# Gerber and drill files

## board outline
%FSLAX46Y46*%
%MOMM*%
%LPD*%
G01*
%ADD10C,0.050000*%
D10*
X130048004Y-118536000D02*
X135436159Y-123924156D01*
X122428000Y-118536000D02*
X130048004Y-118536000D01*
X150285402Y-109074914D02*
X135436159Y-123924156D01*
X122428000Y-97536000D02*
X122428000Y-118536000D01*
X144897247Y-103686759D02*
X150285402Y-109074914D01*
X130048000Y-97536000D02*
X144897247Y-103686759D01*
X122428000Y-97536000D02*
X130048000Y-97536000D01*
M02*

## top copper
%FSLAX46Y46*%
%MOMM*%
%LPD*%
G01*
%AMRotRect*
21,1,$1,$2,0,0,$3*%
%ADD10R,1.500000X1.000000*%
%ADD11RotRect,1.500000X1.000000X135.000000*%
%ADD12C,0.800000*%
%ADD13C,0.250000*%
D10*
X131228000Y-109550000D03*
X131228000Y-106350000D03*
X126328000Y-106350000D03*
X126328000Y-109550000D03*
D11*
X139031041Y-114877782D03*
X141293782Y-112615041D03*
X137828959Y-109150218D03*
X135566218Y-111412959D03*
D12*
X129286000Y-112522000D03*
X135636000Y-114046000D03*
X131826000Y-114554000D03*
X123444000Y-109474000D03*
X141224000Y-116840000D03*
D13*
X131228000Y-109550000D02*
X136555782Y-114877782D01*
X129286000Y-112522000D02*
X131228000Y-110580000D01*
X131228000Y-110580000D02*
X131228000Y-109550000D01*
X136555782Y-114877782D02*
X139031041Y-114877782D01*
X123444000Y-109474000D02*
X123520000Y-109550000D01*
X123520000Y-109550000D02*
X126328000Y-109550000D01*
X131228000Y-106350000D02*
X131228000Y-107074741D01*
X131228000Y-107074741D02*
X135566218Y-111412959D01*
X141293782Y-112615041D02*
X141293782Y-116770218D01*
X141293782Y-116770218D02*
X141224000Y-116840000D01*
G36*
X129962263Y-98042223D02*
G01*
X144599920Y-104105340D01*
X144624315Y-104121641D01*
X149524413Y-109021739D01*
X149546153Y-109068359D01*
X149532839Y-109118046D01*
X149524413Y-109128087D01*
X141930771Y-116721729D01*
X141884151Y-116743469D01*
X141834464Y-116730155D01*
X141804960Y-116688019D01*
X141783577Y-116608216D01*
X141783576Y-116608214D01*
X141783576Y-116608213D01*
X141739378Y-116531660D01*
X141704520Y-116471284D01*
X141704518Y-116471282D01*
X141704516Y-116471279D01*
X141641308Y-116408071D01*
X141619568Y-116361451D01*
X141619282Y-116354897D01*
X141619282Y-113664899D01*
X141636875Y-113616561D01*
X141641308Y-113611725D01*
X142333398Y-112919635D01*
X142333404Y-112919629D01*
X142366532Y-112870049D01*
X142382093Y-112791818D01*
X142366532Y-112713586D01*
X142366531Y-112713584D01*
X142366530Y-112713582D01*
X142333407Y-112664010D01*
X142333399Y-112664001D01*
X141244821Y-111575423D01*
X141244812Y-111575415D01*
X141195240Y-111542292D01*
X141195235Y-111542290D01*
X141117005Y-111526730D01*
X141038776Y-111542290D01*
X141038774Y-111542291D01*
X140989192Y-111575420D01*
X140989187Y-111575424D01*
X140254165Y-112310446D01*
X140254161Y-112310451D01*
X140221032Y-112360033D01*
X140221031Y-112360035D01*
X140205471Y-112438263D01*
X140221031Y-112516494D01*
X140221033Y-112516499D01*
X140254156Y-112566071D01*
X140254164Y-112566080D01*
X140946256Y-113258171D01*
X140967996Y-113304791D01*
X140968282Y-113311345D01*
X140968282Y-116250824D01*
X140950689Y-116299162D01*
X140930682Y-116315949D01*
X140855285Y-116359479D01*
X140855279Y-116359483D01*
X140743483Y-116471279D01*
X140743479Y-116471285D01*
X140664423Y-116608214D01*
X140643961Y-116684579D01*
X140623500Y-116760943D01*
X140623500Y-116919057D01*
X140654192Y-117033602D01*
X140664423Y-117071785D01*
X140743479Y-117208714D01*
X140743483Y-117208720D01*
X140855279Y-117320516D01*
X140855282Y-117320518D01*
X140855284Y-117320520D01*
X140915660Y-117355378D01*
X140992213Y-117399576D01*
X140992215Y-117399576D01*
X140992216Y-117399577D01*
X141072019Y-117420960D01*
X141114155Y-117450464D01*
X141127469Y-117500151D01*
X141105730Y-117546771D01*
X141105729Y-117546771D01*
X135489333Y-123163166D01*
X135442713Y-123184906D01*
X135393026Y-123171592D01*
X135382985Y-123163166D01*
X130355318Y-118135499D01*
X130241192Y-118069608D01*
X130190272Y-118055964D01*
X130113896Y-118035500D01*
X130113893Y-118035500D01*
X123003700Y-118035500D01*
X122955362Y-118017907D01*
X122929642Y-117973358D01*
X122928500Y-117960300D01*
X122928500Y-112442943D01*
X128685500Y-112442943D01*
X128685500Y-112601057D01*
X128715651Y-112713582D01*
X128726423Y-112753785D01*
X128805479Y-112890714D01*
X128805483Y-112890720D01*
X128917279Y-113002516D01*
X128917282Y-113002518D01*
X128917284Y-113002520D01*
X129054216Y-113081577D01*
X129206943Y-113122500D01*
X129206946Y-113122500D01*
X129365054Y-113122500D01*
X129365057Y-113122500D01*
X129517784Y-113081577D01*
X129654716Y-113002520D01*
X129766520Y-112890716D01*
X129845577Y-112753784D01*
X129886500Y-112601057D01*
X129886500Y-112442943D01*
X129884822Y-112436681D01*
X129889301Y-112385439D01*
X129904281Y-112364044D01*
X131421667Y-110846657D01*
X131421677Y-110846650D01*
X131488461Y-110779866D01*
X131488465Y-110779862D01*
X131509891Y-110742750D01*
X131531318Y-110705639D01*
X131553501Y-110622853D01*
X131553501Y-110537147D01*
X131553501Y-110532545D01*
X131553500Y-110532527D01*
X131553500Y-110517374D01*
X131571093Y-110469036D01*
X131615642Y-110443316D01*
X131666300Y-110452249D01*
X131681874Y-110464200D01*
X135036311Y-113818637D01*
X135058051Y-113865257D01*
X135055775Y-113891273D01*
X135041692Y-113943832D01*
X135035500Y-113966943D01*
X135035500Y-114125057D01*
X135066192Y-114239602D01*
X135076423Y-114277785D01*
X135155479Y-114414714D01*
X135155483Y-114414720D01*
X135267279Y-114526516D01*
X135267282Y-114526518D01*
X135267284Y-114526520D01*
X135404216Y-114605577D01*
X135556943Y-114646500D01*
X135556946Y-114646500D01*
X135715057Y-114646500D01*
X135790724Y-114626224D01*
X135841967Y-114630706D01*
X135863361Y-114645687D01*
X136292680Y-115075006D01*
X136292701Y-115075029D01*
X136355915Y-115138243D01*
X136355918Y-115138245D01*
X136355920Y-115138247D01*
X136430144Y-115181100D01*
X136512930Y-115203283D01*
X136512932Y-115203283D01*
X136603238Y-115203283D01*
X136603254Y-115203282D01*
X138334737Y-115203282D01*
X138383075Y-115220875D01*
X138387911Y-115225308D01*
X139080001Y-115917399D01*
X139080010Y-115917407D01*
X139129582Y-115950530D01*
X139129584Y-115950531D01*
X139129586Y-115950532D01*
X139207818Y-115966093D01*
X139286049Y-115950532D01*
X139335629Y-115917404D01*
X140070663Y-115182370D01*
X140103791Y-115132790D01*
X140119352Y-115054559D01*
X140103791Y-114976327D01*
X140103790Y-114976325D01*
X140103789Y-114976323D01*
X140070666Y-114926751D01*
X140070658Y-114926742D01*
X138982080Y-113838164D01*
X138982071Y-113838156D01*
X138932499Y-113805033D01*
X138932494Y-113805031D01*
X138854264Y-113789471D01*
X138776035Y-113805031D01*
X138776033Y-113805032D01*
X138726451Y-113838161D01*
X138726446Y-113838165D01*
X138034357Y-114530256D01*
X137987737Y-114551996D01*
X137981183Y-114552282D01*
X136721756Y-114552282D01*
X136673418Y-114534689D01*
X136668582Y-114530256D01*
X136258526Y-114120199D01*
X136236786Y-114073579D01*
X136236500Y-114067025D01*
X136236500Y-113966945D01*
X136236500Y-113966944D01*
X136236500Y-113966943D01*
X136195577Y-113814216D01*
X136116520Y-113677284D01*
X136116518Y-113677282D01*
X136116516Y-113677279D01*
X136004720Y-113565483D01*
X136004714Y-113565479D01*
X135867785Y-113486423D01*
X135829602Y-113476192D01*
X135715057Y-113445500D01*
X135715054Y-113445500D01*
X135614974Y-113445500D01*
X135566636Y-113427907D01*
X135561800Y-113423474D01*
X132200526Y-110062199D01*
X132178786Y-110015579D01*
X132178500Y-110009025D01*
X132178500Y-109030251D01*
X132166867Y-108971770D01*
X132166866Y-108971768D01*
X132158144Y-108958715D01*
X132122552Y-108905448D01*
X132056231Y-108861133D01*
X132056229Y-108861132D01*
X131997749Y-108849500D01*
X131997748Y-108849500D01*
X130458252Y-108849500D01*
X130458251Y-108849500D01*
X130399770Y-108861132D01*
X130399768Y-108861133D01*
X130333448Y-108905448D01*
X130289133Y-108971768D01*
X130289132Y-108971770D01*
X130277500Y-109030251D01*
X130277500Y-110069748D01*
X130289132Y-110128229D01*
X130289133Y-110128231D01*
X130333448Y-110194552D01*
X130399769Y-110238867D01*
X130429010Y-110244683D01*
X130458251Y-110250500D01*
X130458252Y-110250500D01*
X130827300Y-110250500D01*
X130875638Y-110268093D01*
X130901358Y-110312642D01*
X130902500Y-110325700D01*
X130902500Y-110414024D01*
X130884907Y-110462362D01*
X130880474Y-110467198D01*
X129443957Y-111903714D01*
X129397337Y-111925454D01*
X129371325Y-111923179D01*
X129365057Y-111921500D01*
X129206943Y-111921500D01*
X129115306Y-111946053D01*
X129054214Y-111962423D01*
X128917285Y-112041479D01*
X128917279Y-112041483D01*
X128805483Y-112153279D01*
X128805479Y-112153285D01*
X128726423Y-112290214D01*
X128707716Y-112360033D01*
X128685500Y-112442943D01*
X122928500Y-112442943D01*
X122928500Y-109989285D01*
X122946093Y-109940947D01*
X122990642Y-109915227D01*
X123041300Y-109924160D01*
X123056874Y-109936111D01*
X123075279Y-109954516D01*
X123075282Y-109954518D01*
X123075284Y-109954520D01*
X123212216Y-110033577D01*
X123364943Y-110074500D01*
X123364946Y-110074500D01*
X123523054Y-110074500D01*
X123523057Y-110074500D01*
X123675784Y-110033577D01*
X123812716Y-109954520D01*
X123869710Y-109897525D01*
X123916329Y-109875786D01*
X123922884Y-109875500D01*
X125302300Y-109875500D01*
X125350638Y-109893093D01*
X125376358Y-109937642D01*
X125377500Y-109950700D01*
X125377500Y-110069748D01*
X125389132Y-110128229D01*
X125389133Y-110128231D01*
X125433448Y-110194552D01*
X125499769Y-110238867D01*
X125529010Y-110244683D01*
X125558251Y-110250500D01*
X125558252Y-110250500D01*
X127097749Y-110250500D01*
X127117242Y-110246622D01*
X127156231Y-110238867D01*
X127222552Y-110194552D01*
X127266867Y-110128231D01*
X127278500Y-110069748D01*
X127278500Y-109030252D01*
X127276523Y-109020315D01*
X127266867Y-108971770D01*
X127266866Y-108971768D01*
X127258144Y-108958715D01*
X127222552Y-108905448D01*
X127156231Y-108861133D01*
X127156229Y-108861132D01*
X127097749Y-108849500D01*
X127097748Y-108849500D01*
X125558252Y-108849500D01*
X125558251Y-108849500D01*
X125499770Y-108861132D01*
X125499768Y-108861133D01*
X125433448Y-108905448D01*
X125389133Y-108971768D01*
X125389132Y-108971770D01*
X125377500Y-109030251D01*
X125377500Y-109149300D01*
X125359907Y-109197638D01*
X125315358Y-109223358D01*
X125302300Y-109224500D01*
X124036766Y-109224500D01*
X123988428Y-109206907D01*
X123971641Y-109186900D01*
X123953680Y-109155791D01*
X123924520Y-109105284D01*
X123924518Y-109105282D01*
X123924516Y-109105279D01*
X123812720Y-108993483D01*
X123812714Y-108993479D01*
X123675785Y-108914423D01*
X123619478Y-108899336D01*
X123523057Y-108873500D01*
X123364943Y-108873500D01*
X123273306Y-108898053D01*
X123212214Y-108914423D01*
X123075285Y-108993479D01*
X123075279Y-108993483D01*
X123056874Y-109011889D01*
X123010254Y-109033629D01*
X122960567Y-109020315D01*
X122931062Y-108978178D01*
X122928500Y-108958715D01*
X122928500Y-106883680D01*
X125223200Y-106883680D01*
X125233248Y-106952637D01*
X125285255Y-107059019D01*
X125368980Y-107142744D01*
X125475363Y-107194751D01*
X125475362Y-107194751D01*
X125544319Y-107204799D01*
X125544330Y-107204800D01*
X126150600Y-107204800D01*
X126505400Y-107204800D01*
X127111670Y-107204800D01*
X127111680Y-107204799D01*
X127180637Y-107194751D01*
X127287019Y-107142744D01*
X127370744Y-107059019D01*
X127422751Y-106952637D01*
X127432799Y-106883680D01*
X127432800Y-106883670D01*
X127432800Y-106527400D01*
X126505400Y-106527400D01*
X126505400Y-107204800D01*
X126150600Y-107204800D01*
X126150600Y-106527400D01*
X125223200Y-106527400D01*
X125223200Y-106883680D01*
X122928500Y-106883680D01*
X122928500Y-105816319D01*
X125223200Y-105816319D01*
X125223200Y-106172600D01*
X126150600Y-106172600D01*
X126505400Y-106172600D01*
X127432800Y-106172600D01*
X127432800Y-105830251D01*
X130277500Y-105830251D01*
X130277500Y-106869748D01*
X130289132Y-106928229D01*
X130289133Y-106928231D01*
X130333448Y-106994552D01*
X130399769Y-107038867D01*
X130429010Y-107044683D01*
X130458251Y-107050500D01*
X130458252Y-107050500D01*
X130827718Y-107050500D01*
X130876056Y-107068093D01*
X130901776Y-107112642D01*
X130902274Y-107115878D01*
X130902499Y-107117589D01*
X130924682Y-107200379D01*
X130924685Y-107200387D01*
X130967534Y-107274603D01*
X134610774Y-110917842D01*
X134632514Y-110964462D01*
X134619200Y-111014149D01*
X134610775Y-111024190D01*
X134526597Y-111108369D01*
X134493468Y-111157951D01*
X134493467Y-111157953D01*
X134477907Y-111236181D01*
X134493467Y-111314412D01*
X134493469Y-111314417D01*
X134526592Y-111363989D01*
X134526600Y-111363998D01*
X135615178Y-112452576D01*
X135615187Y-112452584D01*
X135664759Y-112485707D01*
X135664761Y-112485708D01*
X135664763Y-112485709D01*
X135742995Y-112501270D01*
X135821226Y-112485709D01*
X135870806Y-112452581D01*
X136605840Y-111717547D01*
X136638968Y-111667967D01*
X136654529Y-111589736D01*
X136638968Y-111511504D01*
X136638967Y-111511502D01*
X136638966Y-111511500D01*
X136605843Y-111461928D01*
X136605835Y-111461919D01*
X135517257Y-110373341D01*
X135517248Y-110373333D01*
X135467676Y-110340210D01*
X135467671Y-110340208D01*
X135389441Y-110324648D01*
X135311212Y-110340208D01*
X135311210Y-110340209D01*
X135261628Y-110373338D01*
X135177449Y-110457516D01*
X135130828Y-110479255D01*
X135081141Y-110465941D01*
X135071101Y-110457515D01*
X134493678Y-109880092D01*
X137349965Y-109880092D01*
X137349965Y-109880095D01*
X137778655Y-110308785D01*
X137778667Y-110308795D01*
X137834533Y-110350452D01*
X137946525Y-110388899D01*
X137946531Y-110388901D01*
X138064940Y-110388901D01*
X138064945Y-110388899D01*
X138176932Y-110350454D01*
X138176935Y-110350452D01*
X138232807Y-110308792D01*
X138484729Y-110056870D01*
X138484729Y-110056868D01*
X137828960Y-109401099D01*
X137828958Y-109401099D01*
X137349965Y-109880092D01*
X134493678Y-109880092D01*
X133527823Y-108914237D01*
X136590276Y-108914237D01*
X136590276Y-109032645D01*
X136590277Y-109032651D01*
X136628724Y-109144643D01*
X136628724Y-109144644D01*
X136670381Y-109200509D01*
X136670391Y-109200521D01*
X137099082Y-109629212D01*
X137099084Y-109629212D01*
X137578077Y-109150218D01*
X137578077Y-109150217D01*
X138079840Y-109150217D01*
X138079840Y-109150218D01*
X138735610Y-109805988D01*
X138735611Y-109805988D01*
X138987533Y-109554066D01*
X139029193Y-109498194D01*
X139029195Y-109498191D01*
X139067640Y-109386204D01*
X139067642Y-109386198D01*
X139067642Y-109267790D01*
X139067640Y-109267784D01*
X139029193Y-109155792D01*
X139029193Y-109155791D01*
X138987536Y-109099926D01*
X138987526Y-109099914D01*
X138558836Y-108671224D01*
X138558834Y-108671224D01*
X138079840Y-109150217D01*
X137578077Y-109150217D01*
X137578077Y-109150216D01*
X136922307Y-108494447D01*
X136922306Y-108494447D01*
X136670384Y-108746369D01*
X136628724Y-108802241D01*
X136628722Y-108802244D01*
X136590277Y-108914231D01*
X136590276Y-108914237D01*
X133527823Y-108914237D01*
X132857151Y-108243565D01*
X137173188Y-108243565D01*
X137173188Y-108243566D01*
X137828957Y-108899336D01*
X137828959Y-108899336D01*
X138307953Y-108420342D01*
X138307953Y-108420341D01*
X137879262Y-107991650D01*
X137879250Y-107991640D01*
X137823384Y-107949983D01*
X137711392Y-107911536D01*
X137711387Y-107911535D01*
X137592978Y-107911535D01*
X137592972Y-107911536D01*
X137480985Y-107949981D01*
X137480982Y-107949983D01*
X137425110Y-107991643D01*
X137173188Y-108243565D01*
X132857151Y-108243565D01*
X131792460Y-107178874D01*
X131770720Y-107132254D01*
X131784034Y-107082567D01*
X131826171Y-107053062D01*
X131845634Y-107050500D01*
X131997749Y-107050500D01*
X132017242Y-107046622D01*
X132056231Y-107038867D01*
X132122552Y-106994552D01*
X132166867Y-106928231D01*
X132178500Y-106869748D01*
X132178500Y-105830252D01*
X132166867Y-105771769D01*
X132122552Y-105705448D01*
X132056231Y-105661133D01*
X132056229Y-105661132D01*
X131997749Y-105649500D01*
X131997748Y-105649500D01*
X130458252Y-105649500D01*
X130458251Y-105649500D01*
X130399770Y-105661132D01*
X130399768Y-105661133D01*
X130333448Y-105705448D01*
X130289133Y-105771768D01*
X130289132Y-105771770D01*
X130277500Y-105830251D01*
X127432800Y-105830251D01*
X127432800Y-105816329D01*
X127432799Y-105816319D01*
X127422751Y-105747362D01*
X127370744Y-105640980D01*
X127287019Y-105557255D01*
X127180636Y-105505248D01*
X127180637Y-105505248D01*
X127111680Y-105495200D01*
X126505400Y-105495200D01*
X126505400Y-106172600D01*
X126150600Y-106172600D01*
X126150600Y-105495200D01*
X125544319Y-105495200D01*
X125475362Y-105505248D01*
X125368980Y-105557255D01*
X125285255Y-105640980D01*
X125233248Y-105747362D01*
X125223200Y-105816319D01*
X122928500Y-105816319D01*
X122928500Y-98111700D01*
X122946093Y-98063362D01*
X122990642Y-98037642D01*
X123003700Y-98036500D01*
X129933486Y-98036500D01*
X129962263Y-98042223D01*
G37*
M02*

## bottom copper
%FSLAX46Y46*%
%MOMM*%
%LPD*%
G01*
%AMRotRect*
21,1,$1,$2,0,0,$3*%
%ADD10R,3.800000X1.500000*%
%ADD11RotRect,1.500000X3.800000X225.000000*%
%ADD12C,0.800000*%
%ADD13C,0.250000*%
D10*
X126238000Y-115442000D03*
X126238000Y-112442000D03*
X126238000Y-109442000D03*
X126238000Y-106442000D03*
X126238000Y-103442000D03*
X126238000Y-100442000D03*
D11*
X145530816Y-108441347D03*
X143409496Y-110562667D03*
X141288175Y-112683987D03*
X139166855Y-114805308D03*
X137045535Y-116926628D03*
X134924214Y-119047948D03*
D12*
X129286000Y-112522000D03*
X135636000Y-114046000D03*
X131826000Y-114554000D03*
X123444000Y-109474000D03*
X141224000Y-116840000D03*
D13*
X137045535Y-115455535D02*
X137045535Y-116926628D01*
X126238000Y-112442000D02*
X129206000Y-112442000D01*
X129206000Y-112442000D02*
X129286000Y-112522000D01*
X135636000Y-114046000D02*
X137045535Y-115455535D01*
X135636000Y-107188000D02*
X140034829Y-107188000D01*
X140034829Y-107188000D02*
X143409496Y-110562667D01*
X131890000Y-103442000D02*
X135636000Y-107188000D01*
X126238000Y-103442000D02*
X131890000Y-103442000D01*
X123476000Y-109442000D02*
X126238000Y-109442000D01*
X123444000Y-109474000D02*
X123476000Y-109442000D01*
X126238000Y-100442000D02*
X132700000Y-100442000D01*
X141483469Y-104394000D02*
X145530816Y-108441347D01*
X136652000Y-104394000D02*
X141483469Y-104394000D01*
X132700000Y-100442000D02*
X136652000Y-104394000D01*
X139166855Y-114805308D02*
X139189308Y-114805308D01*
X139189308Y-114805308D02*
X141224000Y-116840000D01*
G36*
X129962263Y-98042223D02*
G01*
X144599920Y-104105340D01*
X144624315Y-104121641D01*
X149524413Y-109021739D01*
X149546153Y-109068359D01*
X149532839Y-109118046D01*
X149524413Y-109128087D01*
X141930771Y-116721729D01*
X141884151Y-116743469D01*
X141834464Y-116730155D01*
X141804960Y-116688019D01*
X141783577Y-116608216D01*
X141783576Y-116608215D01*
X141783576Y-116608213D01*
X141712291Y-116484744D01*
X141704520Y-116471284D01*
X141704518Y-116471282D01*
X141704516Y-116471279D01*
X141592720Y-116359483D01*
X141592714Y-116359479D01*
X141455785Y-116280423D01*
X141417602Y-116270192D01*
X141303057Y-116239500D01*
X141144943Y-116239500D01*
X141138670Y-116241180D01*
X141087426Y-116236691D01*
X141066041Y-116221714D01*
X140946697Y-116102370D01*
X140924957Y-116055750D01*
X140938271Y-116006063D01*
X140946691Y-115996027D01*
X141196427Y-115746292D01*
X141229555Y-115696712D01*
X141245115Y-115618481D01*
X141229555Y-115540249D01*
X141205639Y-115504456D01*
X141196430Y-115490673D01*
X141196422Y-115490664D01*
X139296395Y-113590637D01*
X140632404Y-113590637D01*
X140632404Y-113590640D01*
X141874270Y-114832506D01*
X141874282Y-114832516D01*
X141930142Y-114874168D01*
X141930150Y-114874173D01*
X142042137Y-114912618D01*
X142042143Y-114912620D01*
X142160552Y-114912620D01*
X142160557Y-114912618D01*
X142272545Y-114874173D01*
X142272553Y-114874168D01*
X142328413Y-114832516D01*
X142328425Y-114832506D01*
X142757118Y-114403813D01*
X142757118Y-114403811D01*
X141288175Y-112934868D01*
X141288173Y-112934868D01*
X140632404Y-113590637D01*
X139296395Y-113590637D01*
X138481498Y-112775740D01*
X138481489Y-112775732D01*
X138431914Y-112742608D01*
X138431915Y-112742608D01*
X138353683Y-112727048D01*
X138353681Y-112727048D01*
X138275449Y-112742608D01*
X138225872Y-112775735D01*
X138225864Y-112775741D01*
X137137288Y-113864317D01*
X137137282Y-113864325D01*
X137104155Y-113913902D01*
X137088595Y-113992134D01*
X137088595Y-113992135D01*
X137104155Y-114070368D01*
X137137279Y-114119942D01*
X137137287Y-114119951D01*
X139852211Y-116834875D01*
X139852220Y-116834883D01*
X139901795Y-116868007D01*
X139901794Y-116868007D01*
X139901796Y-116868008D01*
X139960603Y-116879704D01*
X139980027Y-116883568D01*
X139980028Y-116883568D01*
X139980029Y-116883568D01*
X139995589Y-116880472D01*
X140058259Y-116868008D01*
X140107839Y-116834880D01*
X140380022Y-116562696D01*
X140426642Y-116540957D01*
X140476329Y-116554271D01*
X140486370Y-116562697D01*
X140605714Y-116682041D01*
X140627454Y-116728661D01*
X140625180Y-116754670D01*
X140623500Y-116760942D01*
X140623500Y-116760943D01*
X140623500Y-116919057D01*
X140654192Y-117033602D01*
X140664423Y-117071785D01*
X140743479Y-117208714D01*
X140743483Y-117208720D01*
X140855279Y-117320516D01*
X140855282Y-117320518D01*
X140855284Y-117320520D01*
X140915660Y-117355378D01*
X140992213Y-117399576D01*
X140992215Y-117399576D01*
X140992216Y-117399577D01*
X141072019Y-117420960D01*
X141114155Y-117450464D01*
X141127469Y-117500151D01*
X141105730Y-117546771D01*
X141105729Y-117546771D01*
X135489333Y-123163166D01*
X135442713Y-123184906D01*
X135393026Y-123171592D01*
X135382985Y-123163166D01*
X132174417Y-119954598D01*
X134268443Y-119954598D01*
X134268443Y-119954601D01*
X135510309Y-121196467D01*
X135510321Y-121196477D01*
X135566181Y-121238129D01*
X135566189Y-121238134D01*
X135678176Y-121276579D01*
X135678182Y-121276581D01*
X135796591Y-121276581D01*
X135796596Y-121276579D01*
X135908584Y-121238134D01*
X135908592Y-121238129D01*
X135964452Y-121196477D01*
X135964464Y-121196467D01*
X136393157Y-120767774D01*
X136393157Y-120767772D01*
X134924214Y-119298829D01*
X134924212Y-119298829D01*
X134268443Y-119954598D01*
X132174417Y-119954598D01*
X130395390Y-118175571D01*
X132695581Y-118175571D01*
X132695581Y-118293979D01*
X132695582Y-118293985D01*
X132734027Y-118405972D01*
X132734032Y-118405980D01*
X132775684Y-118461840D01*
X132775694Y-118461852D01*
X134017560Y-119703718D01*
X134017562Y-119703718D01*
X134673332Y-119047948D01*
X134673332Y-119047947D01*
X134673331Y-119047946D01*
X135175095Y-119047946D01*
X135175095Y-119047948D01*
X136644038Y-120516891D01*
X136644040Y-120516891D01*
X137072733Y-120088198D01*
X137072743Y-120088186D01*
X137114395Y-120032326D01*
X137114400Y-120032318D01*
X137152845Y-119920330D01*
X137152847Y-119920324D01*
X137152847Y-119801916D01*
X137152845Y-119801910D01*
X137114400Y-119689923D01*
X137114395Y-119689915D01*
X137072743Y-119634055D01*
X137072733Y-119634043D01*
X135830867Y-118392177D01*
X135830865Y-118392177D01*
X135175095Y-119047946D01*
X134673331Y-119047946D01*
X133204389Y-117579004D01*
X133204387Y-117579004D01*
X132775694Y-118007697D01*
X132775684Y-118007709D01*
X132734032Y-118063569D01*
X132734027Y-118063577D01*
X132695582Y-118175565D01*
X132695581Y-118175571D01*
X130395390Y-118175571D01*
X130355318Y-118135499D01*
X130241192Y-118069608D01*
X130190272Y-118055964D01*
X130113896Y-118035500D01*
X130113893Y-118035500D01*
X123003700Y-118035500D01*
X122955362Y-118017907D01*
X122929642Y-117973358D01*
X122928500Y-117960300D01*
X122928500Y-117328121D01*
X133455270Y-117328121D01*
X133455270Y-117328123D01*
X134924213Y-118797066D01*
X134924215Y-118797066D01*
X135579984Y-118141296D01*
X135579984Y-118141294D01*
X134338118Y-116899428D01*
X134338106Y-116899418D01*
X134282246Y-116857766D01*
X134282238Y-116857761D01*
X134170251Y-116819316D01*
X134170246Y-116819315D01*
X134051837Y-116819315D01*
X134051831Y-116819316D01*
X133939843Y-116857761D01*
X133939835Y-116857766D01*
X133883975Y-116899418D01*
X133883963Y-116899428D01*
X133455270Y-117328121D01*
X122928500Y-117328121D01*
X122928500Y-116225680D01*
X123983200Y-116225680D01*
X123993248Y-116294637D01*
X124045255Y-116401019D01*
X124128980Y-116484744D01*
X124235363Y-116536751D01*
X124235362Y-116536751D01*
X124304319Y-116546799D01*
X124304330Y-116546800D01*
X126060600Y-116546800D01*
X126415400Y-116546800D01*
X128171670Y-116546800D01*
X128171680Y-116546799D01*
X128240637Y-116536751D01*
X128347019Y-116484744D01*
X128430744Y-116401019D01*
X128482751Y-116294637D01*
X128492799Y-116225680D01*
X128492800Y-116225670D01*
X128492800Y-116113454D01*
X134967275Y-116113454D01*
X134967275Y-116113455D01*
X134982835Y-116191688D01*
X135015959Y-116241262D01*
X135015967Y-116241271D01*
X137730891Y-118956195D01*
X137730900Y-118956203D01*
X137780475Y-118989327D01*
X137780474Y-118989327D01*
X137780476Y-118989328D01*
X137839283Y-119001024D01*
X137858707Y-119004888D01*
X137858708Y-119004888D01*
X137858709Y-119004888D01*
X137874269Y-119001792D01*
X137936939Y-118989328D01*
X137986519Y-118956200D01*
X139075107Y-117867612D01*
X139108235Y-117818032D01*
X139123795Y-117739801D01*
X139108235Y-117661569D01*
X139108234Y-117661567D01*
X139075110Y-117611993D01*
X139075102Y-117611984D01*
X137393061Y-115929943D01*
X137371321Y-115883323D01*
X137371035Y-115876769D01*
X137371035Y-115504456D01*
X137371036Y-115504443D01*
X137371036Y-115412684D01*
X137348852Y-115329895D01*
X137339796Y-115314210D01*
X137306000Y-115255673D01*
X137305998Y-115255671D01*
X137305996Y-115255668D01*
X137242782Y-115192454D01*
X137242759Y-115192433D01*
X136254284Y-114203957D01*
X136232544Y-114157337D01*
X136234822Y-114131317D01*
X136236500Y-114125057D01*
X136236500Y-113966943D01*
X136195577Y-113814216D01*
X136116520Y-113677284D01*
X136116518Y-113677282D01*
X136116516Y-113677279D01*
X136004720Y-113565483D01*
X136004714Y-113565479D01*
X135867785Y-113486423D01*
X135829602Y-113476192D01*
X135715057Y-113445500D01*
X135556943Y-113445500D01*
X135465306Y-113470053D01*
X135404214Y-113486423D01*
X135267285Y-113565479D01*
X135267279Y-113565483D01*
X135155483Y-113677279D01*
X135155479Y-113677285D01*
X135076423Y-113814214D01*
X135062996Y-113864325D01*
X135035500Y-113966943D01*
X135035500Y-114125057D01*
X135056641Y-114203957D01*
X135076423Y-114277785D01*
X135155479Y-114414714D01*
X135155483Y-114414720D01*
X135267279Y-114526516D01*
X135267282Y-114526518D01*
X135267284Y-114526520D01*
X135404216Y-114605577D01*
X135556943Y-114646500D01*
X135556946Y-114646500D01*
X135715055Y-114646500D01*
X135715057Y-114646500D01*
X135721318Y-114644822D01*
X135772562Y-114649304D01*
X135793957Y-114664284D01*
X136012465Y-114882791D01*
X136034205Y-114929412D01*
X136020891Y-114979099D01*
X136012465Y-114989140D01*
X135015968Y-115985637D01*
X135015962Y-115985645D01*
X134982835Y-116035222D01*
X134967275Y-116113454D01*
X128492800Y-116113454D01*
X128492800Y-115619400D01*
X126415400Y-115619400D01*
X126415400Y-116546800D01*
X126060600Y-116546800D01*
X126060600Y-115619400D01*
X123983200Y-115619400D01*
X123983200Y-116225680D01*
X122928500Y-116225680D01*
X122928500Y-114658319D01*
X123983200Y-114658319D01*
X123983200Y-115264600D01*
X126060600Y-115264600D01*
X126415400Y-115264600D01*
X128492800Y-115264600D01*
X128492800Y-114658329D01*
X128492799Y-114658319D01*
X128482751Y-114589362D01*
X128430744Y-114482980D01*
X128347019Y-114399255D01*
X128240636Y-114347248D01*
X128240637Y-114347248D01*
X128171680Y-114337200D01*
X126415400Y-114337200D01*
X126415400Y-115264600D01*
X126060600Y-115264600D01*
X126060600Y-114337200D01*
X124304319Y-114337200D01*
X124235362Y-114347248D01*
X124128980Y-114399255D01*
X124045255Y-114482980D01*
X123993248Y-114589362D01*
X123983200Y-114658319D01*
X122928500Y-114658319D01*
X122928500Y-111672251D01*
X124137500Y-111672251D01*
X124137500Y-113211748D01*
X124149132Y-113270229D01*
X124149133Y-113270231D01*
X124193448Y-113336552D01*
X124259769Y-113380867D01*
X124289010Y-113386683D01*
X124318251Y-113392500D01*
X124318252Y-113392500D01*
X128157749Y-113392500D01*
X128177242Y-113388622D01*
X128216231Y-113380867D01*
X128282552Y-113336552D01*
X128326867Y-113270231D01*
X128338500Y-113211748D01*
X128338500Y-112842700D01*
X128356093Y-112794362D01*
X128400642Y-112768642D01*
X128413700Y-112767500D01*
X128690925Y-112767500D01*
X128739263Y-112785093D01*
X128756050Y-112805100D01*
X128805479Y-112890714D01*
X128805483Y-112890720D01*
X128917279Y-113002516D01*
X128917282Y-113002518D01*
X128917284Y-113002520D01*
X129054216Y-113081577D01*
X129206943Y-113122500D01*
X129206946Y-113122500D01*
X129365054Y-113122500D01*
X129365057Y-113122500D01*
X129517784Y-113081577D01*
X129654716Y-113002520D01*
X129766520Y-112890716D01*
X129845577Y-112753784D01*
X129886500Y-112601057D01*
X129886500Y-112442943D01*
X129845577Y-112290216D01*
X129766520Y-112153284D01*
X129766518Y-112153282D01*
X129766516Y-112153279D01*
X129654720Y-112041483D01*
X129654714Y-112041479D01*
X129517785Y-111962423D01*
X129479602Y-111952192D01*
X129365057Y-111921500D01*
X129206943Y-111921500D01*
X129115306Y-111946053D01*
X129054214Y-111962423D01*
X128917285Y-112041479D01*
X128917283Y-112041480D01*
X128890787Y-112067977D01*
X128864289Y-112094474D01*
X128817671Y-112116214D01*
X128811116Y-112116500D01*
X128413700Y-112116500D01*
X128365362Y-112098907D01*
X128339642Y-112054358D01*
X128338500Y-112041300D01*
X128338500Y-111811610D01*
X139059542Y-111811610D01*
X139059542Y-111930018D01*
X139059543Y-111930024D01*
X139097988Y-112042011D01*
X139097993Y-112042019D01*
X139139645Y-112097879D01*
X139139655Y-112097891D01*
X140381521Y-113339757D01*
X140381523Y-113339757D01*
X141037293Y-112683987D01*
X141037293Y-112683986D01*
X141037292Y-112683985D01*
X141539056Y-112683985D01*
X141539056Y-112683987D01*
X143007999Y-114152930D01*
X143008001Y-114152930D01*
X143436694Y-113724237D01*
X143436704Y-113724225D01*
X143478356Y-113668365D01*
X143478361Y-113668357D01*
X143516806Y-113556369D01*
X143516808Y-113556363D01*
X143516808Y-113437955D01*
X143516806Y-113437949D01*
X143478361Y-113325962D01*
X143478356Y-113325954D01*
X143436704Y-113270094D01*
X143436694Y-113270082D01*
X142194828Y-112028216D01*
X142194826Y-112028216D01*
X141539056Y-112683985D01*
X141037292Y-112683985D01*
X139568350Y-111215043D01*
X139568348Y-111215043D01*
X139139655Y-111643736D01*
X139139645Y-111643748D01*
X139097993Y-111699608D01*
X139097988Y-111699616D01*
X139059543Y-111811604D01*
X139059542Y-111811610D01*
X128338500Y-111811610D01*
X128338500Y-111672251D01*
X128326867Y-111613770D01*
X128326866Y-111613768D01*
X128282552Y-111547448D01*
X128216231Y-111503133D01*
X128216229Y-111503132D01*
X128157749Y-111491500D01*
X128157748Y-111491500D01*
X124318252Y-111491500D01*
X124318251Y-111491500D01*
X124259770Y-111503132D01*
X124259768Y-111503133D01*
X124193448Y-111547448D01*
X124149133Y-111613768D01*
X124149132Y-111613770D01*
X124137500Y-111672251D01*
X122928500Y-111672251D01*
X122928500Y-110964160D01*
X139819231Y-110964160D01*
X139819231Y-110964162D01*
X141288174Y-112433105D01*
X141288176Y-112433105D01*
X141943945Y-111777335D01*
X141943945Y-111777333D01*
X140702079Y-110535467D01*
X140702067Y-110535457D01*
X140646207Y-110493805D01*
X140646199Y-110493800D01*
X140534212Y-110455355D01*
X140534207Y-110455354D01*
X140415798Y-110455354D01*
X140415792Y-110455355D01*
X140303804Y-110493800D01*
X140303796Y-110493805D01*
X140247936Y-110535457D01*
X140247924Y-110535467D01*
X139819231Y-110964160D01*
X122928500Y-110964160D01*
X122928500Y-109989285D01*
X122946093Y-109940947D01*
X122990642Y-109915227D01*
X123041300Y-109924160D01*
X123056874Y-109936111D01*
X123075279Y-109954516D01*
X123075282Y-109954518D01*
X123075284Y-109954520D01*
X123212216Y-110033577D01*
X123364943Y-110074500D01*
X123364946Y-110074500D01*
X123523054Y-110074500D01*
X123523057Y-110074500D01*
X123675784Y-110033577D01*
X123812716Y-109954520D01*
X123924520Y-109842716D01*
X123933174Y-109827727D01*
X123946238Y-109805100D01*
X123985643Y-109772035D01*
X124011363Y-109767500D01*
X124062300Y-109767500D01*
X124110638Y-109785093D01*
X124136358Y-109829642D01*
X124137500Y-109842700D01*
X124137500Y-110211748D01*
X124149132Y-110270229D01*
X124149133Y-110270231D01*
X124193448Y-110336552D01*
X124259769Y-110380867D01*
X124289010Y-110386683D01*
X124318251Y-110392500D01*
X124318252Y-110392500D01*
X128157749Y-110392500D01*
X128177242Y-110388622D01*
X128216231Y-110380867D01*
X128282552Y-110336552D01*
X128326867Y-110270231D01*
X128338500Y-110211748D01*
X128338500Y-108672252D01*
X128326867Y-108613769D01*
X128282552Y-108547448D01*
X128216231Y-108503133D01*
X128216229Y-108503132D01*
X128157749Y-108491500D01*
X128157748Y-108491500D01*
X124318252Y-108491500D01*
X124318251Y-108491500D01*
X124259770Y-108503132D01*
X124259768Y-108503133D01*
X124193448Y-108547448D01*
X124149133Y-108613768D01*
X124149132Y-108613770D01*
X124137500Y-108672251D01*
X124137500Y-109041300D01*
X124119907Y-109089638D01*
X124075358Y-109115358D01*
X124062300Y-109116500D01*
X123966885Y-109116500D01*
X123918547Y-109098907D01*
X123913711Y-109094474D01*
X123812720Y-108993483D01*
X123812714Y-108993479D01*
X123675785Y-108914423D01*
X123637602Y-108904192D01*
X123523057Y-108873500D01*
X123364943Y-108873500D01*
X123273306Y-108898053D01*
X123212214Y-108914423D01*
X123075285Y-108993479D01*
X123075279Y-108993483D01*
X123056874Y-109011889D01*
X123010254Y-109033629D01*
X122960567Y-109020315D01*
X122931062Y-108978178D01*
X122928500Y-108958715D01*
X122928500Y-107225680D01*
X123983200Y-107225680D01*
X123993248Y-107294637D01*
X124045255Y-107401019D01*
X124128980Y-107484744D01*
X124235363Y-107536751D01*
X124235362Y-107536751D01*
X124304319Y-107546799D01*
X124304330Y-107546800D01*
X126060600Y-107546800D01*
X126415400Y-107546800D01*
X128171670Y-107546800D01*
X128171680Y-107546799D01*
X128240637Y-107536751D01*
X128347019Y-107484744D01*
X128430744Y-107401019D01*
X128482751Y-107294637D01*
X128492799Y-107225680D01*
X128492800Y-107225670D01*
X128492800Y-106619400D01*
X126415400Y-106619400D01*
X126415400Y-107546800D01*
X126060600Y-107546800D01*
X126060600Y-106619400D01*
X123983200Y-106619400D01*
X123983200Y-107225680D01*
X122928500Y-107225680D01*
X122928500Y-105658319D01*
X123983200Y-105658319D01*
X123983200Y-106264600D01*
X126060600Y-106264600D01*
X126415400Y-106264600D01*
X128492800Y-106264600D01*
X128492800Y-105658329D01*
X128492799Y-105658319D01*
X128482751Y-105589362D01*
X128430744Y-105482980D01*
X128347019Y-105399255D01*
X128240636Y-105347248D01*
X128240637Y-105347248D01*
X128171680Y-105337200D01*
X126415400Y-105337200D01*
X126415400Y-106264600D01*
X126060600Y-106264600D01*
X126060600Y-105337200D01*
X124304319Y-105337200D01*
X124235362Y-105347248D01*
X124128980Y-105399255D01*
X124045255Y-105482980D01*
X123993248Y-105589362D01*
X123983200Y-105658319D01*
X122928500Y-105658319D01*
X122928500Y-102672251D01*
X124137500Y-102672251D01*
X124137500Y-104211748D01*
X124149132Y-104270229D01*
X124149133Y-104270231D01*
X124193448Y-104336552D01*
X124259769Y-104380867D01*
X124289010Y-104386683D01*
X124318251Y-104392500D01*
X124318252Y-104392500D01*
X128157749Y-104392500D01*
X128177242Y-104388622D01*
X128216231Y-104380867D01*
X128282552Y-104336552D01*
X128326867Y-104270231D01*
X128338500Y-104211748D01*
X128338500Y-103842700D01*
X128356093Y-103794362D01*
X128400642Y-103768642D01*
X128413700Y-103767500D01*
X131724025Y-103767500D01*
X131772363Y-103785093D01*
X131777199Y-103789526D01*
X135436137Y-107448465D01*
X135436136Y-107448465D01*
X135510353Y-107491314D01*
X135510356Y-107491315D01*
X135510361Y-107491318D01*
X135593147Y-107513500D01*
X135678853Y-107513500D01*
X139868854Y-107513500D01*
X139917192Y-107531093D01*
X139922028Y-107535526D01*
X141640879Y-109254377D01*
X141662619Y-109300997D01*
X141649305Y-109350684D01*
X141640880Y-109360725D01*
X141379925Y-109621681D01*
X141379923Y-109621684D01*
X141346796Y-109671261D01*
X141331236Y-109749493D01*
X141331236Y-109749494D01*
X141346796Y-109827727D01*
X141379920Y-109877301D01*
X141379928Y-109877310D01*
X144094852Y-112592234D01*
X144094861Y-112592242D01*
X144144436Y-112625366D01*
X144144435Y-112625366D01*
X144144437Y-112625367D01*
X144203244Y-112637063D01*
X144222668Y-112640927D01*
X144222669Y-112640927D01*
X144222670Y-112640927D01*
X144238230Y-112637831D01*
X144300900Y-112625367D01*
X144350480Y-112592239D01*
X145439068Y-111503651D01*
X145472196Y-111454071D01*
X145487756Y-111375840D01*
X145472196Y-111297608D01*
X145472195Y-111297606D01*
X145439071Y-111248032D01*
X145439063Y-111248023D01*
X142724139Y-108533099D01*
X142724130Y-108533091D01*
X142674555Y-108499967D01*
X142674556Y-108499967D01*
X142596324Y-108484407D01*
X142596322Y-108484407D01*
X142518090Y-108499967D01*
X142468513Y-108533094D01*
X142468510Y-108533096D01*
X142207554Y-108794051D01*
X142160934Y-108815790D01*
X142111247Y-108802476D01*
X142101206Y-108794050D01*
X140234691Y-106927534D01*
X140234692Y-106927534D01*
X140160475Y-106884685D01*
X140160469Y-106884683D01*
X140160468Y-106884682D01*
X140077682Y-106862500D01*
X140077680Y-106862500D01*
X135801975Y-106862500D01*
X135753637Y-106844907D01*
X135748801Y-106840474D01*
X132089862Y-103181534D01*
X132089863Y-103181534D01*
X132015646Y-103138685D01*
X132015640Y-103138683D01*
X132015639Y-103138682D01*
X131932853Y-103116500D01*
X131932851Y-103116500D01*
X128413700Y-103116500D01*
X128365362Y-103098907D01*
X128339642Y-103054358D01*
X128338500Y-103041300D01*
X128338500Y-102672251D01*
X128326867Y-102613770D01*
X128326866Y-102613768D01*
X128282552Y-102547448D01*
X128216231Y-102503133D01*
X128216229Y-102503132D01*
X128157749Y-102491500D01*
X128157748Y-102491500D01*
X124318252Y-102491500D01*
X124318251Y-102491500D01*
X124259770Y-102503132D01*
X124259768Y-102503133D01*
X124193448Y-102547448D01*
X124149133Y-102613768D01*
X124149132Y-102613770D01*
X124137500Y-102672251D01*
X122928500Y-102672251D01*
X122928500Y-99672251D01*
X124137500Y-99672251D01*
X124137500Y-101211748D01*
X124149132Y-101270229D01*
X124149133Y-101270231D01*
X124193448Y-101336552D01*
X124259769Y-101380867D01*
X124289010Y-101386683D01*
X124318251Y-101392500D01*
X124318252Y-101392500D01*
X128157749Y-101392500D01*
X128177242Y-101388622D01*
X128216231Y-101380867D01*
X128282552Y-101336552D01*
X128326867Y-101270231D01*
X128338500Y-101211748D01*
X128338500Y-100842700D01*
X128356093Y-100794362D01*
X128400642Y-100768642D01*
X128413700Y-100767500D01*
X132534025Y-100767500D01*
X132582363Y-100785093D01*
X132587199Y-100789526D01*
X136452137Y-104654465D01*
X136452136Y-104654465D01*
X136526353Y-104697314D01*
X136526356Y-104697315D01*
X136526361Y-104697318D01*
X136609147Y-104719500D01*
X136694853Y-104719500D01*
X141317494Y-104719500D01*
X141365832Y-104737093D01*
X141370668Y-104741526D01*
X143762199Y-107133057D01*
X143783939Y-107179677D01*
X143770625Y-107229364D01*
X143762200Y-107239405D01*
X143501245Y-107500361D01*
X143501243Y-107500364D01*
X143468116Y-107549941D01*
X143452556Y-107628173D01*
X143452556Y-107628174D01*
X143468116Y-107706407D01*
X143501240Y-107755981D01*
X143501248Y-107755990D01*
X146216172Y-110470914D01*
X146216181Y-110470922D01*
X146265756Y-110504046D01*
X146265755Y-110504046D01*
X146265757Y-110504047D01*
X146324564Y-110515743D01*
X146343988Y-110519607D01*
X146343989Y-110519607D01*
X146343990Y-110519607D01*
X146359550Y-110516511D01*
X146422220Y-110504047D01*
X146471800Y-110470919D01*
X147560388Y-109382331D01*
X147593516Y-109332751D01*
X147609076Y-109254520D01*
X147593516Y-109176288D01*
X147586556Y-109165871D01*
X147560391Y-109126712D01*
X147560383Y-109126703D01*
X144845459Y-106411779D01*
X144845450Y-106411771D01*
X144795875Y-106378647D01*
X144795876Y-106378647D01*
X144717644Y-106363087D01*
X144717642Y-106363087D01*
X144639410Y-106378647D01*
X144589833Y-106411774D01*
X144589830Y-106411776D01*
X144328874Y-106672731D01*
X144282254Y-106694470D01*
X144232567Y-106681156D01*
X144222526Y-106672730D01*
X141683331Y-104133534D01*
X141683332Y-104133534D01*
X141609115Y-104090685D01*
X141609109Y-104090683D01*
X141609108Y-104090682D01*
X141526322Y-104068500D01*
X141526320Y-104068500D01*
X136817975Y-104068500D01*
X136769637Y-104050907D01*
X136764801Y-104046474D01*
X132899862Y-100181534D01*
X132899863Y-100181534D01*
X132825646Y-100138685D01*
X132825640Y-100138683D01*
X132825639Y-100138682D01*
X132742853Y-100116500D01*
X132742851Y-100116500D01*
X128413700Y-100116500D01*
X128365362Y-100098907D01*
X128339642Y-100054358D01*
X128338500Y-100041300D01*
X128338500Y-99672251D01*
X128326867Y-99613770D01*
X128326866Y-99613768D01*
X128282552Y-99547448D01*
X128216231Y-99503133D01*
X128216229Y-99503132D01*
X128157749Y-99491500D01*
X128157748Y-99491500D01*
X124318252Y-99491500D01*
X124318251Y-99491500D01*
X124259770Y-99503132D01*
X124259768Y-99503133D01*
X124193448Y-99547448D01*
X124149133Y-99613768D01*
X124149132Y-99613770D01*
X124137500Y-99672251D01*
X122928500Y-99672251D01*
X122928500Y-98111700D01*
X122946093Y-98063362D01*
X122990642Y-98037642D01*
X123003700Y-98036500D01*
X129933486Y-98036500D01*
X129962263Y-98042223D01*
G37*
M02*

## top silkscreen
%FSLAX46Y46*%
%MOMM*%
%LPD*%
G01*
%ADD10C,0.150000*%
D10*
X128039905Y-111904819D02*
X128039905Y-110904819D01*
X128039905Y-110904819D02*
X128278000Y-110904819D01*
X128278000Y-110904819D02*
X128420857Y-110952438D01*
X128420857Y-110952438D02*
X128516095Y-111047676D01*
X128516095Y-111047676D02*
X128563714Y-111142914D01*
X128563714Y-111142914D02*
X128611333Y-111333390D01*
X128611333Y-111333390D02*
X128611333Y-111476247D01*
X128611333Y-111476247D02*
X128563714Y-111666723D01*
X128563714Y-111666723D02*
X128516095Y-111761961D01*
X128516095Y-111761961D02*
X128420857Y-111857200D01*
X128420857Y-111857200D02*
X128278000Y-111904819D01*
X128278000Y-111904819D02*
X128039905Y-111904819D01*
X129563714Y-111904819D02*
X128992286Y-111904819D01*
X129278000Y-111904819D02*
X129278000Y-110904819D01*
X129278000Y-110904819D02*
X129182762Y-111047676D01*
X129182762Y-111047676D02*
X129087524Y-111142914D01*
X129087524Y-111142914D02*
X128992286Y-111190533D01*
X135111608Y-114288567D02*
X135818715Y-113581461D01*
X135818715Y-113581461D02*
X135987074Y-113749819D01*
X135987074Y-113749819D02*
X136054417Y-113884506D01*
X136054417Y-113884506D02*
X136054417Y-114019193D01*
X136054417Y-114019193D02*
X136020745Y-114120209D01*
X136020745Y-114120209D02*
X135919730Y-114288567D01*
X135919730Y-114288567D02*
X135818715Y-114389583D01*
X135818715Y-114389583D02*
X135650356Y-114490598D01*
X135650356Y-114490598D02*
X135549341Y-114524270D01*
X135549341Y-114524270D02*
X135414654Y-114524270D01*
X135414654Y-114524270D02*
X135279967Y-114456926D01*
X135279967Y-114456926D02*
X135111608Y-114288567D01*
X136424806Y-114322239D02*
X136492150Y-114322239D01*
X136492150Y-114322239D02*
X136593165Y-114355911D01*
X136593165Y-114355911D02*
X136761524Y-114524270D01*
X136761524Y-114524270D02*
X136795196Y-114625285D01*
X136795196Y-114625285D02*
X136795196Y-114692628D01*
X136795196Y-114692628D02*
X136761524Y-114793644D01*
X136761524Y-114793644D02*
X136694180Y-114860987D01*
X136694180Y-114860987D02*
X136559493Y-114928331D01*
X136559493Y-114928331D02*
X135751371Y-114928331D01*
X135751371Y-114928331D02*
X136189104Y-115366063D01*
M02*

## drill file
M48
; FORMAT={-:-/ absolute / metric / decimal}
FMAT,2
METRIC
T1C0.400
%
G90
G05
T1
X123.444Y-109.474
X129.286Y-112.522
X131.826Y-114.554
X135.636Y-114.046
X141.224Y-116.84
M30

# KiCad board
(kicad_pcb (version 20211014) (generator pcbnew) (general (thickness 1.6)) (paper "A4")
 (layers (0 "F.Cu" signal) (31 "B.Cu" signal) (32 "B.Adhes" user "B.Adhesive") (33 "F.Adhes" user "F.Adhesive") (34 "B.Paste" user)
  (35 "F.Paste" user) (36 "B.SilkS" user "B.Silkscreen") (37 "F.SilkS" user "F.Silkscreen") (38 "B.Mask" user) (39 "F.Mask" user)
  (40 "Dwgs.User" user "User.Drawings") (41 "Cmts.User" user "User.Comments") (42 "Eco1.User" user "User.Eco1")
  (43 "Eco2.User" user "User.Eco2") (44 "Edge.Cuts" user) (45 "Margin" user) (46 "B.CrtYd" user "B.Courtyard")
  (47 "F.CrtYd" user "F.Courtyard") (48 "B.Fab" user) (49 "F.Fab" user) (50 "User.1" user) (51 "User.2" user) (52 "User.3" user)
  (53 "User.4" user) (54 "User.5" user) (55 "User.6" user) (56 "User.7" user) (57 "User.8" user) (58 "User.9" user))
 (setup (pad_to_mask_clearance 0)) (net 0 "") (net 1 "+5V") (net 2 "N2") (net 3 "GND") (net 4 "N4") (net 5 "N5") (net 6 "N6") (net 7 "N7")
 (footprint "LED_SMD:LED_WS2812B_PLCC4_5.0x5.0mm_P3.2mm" (layer "F.Cu") (at 128.778 107.95 180)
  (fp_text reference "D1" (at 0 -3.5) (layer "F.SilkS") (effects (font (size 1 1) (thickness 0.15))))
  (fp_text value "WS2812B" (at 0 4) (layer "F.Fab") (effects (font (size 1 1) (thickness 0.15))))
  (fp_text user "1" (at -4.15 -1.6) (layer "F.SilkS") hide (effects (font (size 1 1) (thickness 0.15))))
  (pad "1" smd rect (at -2.45 -1.6 180) (size 1.5 1) (layers "F.Cu" "F.Paste" "F.Mask") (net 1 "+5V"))
  (pad "2" smd rect (at -2.45 1.6 180) (size 1.5 1) (layers "F.Cu" "F.Paste" "F.Mask") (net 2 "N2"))
  (pad "3" smd rect (at 2.45 1.6 180) (size 1.5 1) (layers "F.Cu" "F.Paste" "F.Mask") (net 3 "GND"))
  (pad "4" smd rect (at 2.45 -1.6 180) (size 1.5 1) (layers "F.Cu" "F.Paste" "F.Mask") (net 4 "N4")))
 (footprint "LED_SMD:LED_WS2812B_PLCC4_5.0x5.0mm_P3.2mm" (layer "F.Cu") (at 138.43 112.014 135)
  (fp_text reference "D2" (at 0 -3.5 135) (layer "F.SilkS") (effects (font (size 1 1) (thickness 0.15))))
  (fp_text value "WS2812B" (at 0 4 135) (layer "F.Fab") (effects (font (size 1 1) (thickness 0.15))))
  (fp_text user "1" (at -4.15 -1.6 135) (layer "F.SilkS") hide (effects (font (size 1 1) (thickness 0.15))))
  (pad "1" smd rect (at -2.45 -1.6 135) (size 1.5 1) (layers "F.Cu" "F.Paste" "F.Mask") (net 1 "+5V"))
  (pad "2" smd rect (at -2.45 1.6 135) (size 1.5 1) (layers "F.Cu" "F.Paste" "F.Mask") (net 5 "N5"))
  (pad "3" smd rect (at 2.45 1.6 135) (size 1.5 1) (layers "F.Cu" "F.Paste" "F.Mask") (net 3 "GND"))
  (pad "4" smd rect (at 2.45 -1.6 135) (size 1.5 1) (layers "F.Cu" "F.Paste" "F.Mask") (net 2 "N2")))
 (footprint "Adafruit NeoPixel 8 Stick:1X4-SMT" (layer "B.Cu") (at 126.873 107.442 90)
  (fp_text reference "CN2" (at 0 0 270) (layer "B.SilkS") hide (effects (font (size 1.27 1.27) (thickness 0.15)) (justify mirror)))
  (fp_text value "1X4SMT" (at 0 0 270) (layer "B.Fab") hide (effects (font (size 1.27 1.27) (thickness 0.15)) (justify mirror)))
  (pad "1" smd rect (at -8 -0.635 90) (size 1.5 3.8) (layers "B.Cu" "B.Paste" "B.Mask") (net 3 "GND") (solder_mask_margin 0.1016))
  (pad "2" smd rect (at -5 -0.635 90) (size 1.5 3.8) (layers "B.Cu" "B.Paste" "B.Mask") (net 1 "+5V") (solder_mask_margin 0.1016))
  (pad "3" smd rect (at -2 -0.635 90) (size 1.5 3.8) (layers "B.Cu" "B.Paste" "B.Mask") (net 4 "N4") (solder_mask_margin 0.1016))
  (pad "4" smd rect (at 1 -0.635 90) (size 1.5 3.8) (layers "B.Cu" "B.Paste" "B.Mask") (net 3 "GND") (solder_mask_margin 0.1016))
  (pad "5" smd rect (at 4 -0.635 90) (size 1.5 3.8) (layers "B.Cu" "B.Paste" "B.Mask") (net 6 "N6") (solder_mask_margin 0.1016))
  (pad "6" smd rect (at 7 -0.635 90) (size 1.5 3.8) (layers "B.Cu" "B.Paste" "B.Mask") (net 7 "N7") (solder_mask_margin 0.1016)))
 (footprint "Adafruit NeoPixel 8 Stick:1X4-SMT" (layer "B.Cu") (at 139.424949 113.649188 -135)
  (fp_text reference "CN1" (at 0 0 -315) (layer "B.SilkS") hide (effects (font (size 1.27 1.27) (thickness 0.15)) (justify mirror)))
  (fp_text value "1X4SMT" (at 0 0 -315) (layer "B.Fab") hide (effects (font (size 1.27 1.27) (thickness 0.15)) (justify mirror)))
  (pad "1" smd rect (at -8 -0.635 225) (size 1.5 3.8) (layers "B.Cu" "B.Paste" "B.Mask") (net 7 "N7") (solder_mask_margin 0.1016))
  (pad "2" smd rect (at -5 -0.635 225) (size 1.5 3.8) (layers "B.Cu" "B.Paste" "B.Mask") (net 6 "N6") (solder_mask_margin 0.1016))
  (pad "3" smd rect (at -2 -0.635 225) (size 1.5 3.8) (layers "B.Cu" "B.Paste" "B.Mask") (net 3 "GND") (solder_mask_margin 0.1016))
  (pad "4" smd rect (at 1 -0.635 225) (size 1.5 3.8) (layers "B.Cu" "B.Paste" "B.Mask") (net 5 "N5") (solder_mask_margin 0.1016))
  (pad "5" smd rect (at 4 -0.635 225) (size 1.5 3.8) (layers "B.Cu" "B.Paste" "B.Mask") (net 1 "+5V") (solder_mask_margin 0.1016))
  (pad "6" smd rect (at 7 -0.635 225) (size 1.5 3.8) (layers "B.Cu" "B.Paste" "B.Mask") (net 3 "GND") (solder_mask_margin 0.1016)))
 (gr_line locked (start 130.048004 118.536) (end 135.436159 123.924156) (layer "Edge.Cuts") (width 0.05))
 (gr_line (start 122.428 118.536) (end 130.048004 118.536) (layer "Edge.Cuts") (width 0.05))
 (gr_line (start 150.285402 109.074914) (end 135.436159 123.924156) (layer "Edge.Cuts") (width 0.05))
 (gr_line (start 122.428 97.536) (end 122.428 118.536) (layer "Edge.Cuts") (width 0.05))
 (gr_line (start 144.897247 103.686759) (end 150.285402 109.074914) (layer "Edge.Cuts") (width 0.05))
 (gr_line (start 130.048 97.536) (end 144.897247 103.686759) (layer "Edge.Cuts") (width 0.05))
 (gr_line (start 122.428 97.536) (end 130.048 97.536) (layer "Edge.Cuts") (width 0.05))
 (segment (start 131.228 109.55) (end 136.555782 114.877782) (width 0.25) (layer "F.Cu") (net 1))
 (segment (start 129.286 112.522) (end 131.228 110.58) (width 0.25) (layer "F.Cu") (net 1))
 (segment (start 131.228 110.58) (end 131.228 109.55) (width 0.25) (layer "F.Cu") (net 1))
 (segment (start 136.555782 114.877782) (end 139.031041 114.877782) (width 0.25) (layer "F.Cu") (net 1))
 (via (at 129.286 112.522) (size 0.8) (drill 0.4) (layers "F.Cu" "B.Cu") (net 1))
 (via (at 135.636 114.046) (size 0.8) (drill 0.4) (layers "F.Cu" "B.Cu") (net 1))
 (segment (start 137.045535 115.455535) (end 137.045535 116.926628) (width 0.25) (layer "B.Cu") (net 1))
 (segment (start 126.238 112.442) (end 129.206 112.442) (width 0.25) (layer "B.Cu") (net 1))
 (segment (start 129.206 112.442) (end 129.286 112.522) (width 0.25) (layer "B.Cu") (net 1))
 (segment (start 135.636 114.046) (end 137.045535 115.455535) (width 0.25) (layer "B.Cu") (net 1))
 (via (at 131.826 114.554) (size 0.8) (drill 0.4) (layers "F.Cu" "B.Cu") (free) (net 3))
 (segment (start 135.636 107.188) (end 140.034829 107.188) (width 0.25) (layer "B.Cu") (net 6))
 (segment (start 140.034829 107.188) (end 143.409496 110.562667) (width 0.25) (layer "B.Cu") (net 6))
 (segment (start 131.89 103.442) (end 135.636 107.188) (width 0.25) (layer "B.Cu") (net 6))
 (segment (start 126.238 103.442) (end 131.89 103.442) (width 0.25) (layer "B.Cu") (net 6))
 (segment (start 123.444 109.474) (end 123.52 109.55) (width 0.25) (layer "F.Cu") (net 4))
 (segment (start 123.52 109.55) (end 126.328 109.55) (width 0.25) (layer "F.Cu") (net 4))
 (via (at 123.444 109.474) (size 0.8) (drill 0.4) (layers "F.Cu" "B.Cu") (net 4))
 (segment (start 123.476 109.442) (end 126.238 109.442) (width 0.25) (layer "B.Cu") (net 4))
 (segment (start 123.444 109.474) (end 123.476 109.442) (width 0.25) (layer "B.Cu") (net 4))
 (segment (start 131.228 106.35) (end 131.228 107.074741) (width 0.25) (layer "F.Cu") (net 2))
 (segment (start 131.228 107.074741) (end 135.566218 111.412959) (width 0.25) (layer "F.Cu") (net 2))
 (segment (start 126.238 100.442) (end 132.7 100.442) (width 0.25) (layer "B.Cu") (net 7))
 (segment (start 141.483469 104.394) (end 145.530816 108.441347) (width 0.25) (layer "B.Cu") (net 7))
 (segment (start 136.652 104.394) (end 141.483469 104.394) (width 0.25) (layer "B.Cu") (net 7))
 (segment (start 132.7 100.442) (end 136.652 104.394) (width 0.25) (layer "B.Cu") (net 7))
 (segment (start 141.293782 112.615041) (end 141.293782 116.770218) (width 0.25) (layer "F.Cu") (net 5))
 (segment (start 141.293782 116.770218) (end 141.224 116.84) (width 0.25) (layer "F.Cu") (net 5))
 (via (at 141.224 116.84) (size 0.8) (drill 0.4) (layers "F.Cu" "B.Cu") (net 5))
 (segment (start 139.166855 114.805308) (end 139.189308 114.805308) (width 0.25) (layer "B.Cu") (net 5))
 (segment (start 139.189308 114.805308) (end 141.224 116.84) (width 0.25) (layer "B.Cu") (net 5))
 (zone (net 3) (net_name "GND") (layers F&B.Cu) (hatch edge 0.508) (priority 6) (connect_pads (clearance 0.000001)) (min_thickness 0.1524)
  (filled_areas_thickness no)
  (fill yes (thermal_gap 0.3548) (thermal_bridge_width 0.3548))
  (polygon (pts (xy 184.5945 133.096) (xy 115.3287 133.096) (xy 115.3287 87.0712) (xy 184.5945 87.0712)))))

